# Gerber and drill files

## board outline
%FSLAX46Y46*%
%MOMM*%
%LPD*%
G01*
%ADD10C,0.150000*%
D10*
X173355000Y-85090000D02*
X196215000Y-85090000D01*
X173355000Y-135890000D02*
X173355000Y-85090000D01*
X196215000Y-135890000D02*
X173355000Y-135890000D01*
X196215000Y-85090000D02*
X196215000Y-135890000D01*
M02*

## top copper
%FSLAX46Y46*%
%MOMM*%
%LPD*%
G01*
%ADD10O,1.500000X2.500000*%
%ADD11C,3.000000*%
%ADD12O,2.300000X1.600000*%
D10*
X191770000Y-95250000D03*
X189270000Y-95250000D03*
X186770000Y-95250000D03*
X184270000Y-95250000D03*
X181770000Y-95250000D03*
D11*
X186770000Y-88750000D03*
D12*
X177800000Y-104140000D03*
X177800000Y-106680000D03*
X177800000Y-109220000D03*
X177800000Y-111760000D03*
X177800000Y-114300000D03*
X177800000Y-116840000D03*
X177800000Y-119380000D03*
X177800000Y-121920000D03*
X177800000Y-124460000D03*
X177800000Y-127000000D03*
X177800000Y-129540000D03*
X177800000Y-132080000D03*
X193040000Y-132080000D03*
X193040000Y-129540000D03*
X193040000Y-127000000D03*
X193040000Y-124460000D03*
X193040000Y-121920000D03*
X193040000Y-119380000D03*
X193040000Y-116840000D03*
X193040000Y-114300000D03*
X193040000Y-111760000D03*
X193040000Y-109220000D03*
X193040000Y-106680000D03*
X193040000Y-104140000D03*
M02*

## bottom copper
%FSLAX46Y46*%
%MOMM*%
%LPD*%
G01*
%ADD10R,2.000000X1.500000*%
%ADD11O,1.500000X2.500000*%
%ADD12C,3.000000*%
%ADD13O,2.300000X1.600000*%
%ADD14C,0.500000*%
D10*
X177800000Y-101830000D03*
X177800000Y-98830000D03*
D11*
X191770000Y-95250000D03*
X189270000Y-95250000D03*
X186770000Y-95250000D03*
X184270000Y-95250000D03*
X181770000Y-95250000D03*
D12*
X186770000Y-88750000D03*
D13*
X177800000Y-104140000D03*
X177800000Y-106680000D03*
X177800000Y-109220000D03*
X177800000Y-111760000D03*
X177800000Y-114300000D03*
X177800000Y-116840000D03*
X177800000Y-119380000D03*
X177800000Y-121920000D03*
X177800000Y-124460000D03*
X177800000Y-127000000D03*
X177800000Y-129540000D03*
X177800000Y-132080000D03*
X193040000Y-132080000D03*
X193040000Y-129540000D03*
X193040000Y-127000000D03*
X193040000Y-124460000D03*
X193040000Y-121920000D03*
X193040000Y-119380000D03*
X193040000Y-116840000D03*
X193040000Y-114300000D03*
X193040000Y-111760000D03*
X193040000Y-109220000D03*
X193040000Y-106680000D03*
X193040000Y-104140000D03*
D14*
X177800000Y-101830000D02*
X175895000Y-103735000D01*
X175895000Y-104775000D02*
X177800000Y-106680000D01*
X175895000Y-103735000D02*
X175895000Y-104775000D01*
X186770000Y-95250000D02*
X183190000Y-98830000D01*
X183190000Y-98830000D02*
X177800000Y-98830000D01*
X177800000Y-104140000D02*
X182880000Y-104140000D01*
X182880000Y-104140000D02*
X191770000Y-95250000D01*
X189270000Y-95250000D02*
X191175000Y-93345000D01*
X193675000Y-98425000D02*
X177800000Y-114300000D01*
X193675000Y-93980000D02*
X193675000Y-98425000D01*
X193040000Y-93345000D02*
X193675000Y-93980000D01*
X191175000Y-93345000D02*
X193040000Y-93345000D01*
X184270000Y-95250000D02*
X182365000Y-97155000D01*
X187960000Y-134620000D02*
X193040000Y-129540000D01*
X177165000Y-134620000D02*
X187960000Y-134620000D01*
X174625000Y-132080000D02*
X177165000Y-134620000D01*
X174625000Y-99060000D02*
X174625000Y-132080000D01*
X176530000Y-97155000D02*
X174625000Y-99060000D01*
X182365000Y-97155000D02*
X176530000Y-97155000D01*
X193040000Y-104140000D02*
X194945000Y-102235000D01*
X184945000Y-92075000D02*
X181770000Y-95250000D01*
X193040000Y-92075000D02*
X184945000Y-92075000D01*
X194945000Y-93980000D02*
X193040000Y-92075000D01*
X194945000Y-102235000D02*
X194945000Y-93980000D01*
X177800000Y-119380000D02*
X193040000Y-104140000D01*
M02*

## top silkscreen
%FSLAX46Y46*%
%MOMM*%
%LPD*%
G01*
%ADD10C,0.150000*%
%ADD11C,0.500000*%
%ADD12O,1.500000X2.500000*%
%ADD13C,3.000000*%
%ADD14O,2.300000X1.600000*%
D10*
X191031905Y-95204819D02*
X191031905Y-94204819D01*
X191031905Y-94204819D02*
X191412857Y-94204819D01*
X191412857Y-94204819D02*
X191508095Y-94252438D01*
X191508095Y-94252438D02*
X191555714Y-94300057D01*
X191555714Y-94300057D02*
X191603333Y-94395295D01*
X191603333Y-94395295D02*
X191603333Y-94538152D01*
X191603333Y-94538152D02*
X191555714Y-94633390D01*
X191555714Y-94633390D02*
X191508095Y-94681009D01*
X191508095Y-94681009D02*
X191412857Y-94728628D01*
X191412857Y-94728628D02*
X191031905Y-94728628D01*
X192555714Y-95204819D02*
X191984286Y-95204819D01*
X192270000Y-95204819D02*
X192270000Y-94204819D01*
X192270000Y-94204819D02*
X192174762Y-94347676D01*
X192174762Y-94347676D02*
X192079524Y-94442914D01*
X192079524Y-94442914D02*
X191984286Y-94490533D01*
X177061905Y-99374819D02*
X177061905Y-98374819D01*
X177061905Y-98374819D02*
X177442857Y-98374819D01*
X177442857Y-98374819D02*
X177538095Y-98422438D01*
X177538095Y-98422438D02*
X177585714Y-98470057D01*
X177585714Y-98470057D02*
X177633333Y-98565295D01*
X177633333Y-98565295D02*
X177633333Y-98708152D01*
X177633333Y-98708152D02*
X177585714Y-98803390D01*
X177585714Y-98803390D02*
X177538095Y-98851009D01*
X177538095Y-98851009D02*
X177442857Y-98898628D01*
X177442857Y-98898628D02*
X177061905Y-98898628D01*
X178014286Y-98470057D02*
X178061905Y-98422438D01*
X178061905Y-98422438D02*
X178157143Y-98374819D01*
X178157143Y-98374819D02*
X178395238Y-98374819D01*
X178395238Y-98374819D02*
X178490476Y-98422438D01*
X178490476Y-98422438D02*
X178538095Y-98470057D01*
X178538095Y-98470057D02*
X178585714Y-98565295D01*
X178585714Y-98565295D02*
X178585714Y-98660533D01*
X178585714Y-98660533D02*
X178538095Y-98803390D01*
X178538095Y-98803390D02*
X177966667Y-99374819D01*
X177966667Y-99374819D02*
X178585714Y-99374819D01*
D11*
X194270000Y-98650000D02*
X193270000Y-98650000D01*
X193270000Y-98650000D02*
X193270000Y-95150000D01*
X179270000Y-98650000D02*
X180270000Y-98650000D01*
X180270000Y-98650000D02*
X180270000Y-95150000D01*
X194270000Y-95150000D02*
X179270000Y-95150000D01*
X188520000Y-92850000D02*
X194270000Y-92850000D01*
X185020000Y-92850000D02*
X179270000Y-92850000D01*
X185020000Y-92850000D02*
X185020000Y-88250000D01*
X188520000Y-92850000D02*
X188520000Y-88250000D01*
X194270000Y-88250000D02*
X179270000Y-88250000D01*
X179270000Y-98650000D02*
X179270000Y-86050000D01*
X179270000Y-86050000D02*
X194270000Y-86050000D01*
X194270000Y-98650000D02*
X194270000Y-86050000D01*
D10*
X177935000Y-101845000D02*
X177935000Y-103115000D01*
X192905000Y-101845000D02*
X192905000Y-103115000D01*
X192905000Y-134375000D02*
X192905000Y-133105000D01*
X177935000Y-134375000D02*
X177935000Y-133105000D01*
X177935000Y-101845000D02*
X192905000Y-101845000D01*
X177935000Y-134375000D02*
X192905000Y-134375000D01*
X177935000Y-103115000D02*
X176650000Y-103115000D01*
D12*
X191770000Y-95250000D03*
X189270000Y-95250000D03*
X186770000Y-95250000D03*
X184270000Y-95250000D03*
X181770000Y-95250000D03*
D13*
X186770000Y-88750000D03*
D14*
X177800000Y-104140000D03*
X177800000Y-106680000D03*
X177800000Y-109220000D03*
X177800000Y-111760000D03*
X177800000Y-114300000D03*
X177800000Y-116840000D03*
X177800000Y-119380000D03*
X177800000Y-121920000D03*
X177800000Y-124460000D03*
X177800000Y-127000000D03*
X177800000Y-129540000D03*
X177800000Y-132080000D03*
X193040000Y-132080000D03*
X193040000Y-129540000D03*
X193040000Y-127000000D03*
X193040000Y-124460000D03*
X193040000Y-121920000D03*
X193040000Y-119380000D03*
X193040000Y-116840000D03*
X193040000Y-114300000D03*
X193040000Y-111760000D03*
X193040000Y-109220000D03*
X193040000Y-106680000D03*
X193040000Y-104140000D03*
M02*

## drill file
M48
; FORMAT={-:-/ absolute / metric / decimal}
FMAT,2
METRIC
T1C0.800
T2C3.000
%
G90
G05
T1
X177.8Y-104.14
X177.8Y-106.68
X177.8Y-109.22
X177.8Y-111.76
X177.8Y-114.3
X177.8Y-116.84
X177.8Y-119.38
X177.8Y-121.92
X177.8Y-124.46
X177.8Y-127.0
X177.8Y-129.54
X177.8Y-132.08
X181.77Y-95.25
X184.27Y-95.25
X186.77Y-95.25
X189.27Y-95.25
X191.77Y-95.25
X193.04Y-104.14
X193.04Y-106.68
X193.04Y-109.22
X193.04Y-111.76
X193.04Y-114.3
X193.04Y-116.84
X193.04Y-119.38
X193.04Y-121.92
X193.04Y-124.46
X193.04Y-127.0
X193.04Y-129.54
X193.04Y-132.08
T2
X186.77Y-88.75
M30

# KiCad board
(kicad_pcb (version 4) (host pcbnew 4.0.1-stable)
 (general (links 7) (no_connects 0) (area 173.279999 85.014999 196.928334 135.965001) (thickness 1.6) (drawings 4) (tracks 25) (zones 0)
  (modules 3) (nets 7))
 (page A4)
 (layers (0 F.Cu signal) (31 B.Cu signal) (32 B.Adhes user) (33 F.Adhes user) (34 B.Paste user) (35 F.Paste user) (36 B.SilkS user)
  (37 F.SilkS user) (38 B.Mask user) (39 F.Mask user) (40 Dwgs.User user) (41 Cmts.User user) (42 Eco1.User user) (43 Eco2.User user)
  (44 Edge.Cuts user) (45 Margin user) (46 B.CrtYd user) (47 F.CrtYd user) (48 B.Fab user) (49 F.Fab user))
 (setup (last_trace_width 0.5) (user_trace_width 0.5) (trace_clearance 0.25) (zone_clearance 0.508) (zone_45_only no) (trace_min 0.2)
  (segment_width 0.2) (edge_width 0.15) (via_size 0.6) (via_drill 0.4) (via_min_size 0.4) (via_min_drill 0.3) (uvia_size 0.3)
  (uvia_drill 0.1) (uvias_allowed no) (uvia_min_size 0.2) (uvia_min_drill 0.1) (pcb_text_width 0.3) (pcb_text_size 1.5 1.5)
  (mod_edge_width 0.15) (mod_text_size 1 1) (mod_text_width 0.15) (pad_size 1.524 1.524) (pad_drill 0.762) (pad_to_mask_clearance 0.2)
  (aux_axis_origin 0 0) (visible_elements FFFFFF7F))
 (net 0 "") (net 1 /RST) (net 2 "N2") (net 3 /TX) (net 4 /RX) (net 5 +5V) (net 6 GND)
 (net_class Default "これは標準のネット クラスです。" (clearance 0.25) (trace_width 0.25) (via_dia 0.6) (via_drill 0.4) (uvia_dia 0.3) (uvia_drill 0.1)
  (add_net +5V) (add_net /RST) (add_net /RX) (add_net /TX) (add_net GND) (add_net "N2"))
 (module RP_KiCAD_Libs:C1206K (layer B.Cu) (at 177.8 100.33 90)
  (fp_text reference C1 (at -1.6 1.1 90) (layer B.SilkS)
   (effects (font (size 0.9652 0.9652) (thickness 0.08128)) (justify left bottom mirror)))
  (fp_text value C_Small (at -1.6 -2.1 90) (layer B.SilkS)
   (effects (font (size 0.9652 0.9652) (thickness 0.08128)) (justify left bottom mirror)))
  (pad 1 smd rect (at -1.5 0 90) (size 1.5 2) (layers B.Cu B.Paste B.Mask) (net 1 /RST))
  (pad 2 smd rect (at 1.5 0 90) (size 1.5 2) (layers B.Cu B.Paste B.Mask) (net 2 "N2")))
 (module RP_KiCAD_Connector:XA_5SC (layer F.Cu) (at 191.77 95.25 180)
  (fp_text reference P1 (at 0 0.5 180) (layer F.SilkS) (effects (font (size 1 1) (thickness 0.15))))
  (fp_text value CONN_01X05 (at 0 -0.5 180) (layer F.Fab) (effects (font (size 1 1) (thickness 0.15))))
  (fp_line (start -2.5 -3.4) (end -1.5 -3.4) (layer F.SilkS) (width 0.5))
  (fp_line (start -1.5 -3.4) (end -1.5 0.1) (layer F.SilkS) (width 0.5))
  (fp_line (start 12.5 -3.4) (end 11.5 -3.4) (layer F.SilkS) (width 0.5))
  (fp_line (start 11.5 -3.4) (end 11.5 0.1) (layer F.SilkS) (width 0.5))
  (fp_line (start -2.5 0.1) (end 12.5 0.1) (layer F.SilkS) (width 0.5))
  (fp_line (start 3.25 2.4) (end -2.5 2.4) (layer F.SilkS) (width 0.5))
  (fp_line (start 6.75 2.4) (end 12.5 2.4) (layer F.SilkS) (width 0.5))
  (fp_line (start 6.75 2.4) (end 6.75 7) (layer F.SilkS) (width 0.5))
  (fp_line (start 3.25 2.4) (end 3.25 7) (layer F.SilkS) (width 0.5))
  (fp_line (start -2.5 7) (end 12.5 7) (layer F.SilkS) (width 0.5))
  (fp_line (start 12.5 -3.4) (end 12.5 9.2) (layer F.SilkS) (width 0.5))
  (fp_line (start 12.5 9.2) (end -2.5 9.2) (layer F.SilkS) (width 0.5))
  (fp_line (start -2.5 -3.4) (end -2.5 9.2) (layer F.SilkS) (width 0.5))
  (pad 1 thru_hole oval (at 0 0 180) (size 1.5 2.5) (drill 0.8) (layers *.Cu *.Mask F.SilkS) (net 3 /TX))
  (pad 2 thru_hole oval (at 2.5 0 180) (size 1.5 2.5) (drill 0.8) (layers *.Cu *.Mask F.SilkS) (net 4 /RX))
  (pad 3 thru_hole oval (at 5 0 180) (size 1.5 2.5) (drill 0.8) (layers *.Cu *.Mask F.SilkS) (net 2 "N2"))
  (pad 4 thru_hole oval (at 7.5 0 180) (size 1.5 2.5) (drill 0.8) (layers *.Cu *.Mask F.SilkS) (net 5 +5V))
  (pad 5 thru_hole oval (at 10 0 180) (size 1.5 2.5) (drill 0.8) (layers *.Cu *.Mask F.SilkS) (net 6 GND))
  (pad "" thru_hole circle (at 5 6.5 180) (size 3 3) (drill 3) (layers *.Cu *.Mask F.SilkS) (clearance -0.3)))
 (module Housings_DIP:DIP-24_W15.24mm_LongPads (layer F.Cu) (at 177.8 104.14)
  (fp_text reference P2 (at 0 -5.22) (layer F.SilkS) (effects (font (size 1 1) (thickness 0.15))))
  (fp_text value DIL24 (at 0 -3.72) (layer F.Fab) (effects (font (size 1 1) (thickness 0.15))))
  (fp_line (start 0.135 -2.295) (end 0.135 -1.025) (layer F.SilkS) (width 0.15))
  (fp_line (start 15.105 -2.295) (end 15.105 -1.025) (layer F.SilkS) (width 0.15))
  (fp_line (start 15.105 30.235) (end 15.105 28.965) (layer F.SilkS) (width 0.15))
  (fp_line (start 0.135 30.235) (end 0.135 28.965) (layer F.SilkS) (width 0.15))
  (fp_line (start 0.135 -2.295) (end 15.105 -2.295) (layer F.SilkS) (width 0.15))
  (fp_line (start 0.135 30.235) (end 15.105 30.235) (layer F.SilkS) (width 0.15))
  (fp_line (start 0.135 -1.025) (end -1.15 -1.025) (layer F.SilkS) (width 0.15))
  (pad 1 thru_hole oval (at 0 0) (size 2.3 1.6) (drill 0.8) (layers *.Cu *.Mask F.SilkS) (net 3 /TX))
  (pad 2 thru_hole oval (at 0 2.54) (size 2.3 1.6) (drill 0.8) (layers *.Cu *.Mask F.SilkS) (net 1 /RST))
  (pad 3 thru_hole oval (at 0 5.08) (size 2.3 1.6) (drill 0.8) (layers *.Cu *.Mask F.SilkS))
  (pad 4 thru_hole oval (at 0 7.62) (size 2.3 1.6) (drill 0.8) (layers *.Cu *.Mask F.SilkS))
  (pad 5 thru_hole oval (at 0 10.16) (size 2.3 1.6) (drill 0.8) (layers *.Cu *.Mask F.SilkS) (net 4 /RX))
  (pad 6 thru_hole oval (at 0 12.7) (size 2.3 1.6) (drill 0.8) (layers *.Cu *.Mask F.SilkS))
  (pad 7 thru_hole oval (at 0 15.24) (size 2.3 1.6) (drill 0.8) (layers *.Cu *.Mask F.SilkS) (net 6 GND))
  (pad 8 thru_hole oval (at 0 17.78) (size 2.3 1.6) (drill 0.8) (layers *.Cu *.Mask F.SilkS))
  (pad 9 thru_hole oval (at 0 20.32) (size 2.3 1.6) (drill 0.8) (layers *.Cu *.Mask F.SilkS))
  (pad 10 thru_hole oval (at 0 22.86) (size 2.3 1.6) (drill 0.8) (layers *.Cu *.Mask F.SilkS))
  (pad 11 thru_hole oval (at 0 25.4) (size 2.3 1.6) (drill 0.8) (layers *.Cu *.Mask F.SilkS))
  (pad 12 thru_hole oval (at 0 27.94) (size 2.3 1.6) (drill 0.8) (layers *.Cu *.Mask F.SilkS))
  (pad 13 thru_hole oval (at 15.24 27.94) (size 2.3 1.6) (drill 0.8) (layers *.Cu *.Mask F.SilkS))
  (pad 14 thru_hole oval (at 15.24 25.4) (size 2.3 1.6) (drill 0.8) (layers *.Cu *.Mask F.SilkS) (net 5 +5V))
  (pad 15 thru_hole oval (at 15.24 22.86) (size 2.3 1.6) (drill 0.8) (layers *.Cu *.Mask F.SilkS))
  (pad 16 thru_hole oval (at 15.24 20.32) (size 2.3 1.6) (drill 0.8) (layers *.Cu *.Mask F.SilkS))
  (pad 17 thru_hole oval (at 15.24 17.78) (size 2.3 1.6) (drill 0.8) (layers *.Cu *.Mask F.SilkS))
  (pad 18 thru_hole oval (at 15.24 15.24) (size 2.3 1.6) (drill 0.8) (layers *.Cu *.Mask F.SilkS))
  (pad 19 thru_hole oval (at 15.24 12.7) (size 2.3 1.6) (drill 0.8) (layers *.Cu *.Mask F.SilkS))
  (pad 20 thru_hole oval (at 15.24 10.16) (size 2.3 1.6) (drill 0.8) (layers *.Cu *.Mask F.SilkS))
  (pad 21 thru_hole oval (at 15.24 7.62) (size 2.3 1.6) (drill 0.8) (layers *.Cu *.Mask F.SilkS))
  (pad 22 thru_hole oval (at 15.24 5.08) (size 2.3 1.6) (drill 0.8) (layers *.Cu *.Mask F.SilkS))
  (pad 23 thru_hole oval (at 15.24 2.54) (size 2.3 1.6) (drill 0.8) (layers *.Cu *.Mask F.SilkS))
  (pad 24 thru_hole oval (at 15.24 0) (size 2.3 1.6) (drill 0.8) (layers *.Cu *.Mask F.SilkS) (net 6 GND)))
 (gr_line (start 173.355 85.09) (end 196.215 85.09) (angle 90) (layer Edge.Cuts) (width 0.15))
 (gr_line (start 173.355 135.89) (end 173.355 85.09) (angle 90) (layer Edge.Cuts) (width 0.15))
 (gr_line (start 196.215 135.89) (end 173.355 135.89) (angle 90) (layer Edge.Cuts) (width 0.15))
 (gr_line (start 196.215 85.09) (end 196.215 135.89) (angle 90) (layer Edge.Cuts) (width 0.15))
 (segment (start 177.8 101.83) (end 175.895 103.735) (width 0.5) (layer B.Cu) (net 1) (status 400000))
 (segment (start 175.895 104.775) (end 177.8 106.68) (width 0.5) (layer B.Cu) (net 1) (status 800000))
 (segment (start 175.895 103.735) (end 175.895 104.775) (width 0.5) (layer B.Cu) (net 1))
 (segment (start 186.77 95.25) (end 183.19 98.83) (width 0.5) (layer B.Cu) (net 2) (status 400000))
 (segment (start 183.19 98.83) (end 177.8 98.83) (width 0.5) (layer B.Cu) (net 2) (status 800000))
 (segment (start 177.8 104.14) (end 182.88 104.14) (width 0.5) (layer B.Cu) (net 3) (status 400000))
 (segment (start 182.88 104.14) (end 191.77 95.25) (width 0.5) (layer B.Cu) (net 3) (status 800000))
 (segment (start 189.27 95.25) (end 191.175 93.345) (width 0.5) (layer B.Cu) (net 4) (status 400000))
 (segment (start 193.675 98.425) (end 177.8 114.3) (width 0.5) (layer B.Cu) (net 4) (status 800000))
 (segment (start 193.675 93.98) (end 193.675 98.425) (width 0.5) (layer B.Cu) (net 4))
 (segment (start 193.04 93.345) (end 193.675 93.98) (width 0.5) (layer B.Cu) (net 4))
 (segment (start 191.175 93.345) (end 193.04 93.345) (width 0.5) (layer B.Cu) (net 4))
 (segment (start 184.27 95.25) (end 182.365 97.155) (width 0.5) (layer B.Cu) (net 5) (status 400000))
 (segment (start 187.96 134.62) (end 193.04 129.54) (width 0.5) (layer B.Cu) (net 5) (status 800000))
 (segment (start 177.165 134.62) (end 187.96 134.62) (width 0.5) (layer B.Cu) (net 5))
 (segment (start 174.625 132.08) (end 177.165 134.62) (width 0.5) (layer B.Cu) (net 5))
 (segment (start 174.625 99.06) (end 174.625 132.08) (width 0.5) (layer B.Cu) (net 5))
 (segment (start 176.53 97.155) (end 174.625 99.06) (width 0.5) (layer B.Cu) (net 5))
 (segment (start 182.365 97.155) (end 176.53 97.155) (width 0.5) (layer B.Cu) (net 5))
 (segment (start 193.04 104.14) (end 194.945 102.235) (width 0.5) (layer B.Cu) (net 6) (status 400000))
 (segment (start 184.945 92.075) (end 181.77 95.25) (width 0.5) (layer B.Cu) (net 6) (status 800000))
 (segment (start 193.04 92.075) (end 184.945 92.075) (width 0.5) (layer B.Cu) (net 6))
 (segment (start 194.945 93.98) (end 193.04 92.075) (width 0.5) (layer B.Cu) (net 6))
 (segment (start 194.945 102.235) (end 194.945 93.98) (width 0.5) (layer B.Cu) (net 6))
 (segment (start 177.8 119.38) (end 193.04 104.14) (width 0.5) (layer B.Cu) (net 6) (status C00000)))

